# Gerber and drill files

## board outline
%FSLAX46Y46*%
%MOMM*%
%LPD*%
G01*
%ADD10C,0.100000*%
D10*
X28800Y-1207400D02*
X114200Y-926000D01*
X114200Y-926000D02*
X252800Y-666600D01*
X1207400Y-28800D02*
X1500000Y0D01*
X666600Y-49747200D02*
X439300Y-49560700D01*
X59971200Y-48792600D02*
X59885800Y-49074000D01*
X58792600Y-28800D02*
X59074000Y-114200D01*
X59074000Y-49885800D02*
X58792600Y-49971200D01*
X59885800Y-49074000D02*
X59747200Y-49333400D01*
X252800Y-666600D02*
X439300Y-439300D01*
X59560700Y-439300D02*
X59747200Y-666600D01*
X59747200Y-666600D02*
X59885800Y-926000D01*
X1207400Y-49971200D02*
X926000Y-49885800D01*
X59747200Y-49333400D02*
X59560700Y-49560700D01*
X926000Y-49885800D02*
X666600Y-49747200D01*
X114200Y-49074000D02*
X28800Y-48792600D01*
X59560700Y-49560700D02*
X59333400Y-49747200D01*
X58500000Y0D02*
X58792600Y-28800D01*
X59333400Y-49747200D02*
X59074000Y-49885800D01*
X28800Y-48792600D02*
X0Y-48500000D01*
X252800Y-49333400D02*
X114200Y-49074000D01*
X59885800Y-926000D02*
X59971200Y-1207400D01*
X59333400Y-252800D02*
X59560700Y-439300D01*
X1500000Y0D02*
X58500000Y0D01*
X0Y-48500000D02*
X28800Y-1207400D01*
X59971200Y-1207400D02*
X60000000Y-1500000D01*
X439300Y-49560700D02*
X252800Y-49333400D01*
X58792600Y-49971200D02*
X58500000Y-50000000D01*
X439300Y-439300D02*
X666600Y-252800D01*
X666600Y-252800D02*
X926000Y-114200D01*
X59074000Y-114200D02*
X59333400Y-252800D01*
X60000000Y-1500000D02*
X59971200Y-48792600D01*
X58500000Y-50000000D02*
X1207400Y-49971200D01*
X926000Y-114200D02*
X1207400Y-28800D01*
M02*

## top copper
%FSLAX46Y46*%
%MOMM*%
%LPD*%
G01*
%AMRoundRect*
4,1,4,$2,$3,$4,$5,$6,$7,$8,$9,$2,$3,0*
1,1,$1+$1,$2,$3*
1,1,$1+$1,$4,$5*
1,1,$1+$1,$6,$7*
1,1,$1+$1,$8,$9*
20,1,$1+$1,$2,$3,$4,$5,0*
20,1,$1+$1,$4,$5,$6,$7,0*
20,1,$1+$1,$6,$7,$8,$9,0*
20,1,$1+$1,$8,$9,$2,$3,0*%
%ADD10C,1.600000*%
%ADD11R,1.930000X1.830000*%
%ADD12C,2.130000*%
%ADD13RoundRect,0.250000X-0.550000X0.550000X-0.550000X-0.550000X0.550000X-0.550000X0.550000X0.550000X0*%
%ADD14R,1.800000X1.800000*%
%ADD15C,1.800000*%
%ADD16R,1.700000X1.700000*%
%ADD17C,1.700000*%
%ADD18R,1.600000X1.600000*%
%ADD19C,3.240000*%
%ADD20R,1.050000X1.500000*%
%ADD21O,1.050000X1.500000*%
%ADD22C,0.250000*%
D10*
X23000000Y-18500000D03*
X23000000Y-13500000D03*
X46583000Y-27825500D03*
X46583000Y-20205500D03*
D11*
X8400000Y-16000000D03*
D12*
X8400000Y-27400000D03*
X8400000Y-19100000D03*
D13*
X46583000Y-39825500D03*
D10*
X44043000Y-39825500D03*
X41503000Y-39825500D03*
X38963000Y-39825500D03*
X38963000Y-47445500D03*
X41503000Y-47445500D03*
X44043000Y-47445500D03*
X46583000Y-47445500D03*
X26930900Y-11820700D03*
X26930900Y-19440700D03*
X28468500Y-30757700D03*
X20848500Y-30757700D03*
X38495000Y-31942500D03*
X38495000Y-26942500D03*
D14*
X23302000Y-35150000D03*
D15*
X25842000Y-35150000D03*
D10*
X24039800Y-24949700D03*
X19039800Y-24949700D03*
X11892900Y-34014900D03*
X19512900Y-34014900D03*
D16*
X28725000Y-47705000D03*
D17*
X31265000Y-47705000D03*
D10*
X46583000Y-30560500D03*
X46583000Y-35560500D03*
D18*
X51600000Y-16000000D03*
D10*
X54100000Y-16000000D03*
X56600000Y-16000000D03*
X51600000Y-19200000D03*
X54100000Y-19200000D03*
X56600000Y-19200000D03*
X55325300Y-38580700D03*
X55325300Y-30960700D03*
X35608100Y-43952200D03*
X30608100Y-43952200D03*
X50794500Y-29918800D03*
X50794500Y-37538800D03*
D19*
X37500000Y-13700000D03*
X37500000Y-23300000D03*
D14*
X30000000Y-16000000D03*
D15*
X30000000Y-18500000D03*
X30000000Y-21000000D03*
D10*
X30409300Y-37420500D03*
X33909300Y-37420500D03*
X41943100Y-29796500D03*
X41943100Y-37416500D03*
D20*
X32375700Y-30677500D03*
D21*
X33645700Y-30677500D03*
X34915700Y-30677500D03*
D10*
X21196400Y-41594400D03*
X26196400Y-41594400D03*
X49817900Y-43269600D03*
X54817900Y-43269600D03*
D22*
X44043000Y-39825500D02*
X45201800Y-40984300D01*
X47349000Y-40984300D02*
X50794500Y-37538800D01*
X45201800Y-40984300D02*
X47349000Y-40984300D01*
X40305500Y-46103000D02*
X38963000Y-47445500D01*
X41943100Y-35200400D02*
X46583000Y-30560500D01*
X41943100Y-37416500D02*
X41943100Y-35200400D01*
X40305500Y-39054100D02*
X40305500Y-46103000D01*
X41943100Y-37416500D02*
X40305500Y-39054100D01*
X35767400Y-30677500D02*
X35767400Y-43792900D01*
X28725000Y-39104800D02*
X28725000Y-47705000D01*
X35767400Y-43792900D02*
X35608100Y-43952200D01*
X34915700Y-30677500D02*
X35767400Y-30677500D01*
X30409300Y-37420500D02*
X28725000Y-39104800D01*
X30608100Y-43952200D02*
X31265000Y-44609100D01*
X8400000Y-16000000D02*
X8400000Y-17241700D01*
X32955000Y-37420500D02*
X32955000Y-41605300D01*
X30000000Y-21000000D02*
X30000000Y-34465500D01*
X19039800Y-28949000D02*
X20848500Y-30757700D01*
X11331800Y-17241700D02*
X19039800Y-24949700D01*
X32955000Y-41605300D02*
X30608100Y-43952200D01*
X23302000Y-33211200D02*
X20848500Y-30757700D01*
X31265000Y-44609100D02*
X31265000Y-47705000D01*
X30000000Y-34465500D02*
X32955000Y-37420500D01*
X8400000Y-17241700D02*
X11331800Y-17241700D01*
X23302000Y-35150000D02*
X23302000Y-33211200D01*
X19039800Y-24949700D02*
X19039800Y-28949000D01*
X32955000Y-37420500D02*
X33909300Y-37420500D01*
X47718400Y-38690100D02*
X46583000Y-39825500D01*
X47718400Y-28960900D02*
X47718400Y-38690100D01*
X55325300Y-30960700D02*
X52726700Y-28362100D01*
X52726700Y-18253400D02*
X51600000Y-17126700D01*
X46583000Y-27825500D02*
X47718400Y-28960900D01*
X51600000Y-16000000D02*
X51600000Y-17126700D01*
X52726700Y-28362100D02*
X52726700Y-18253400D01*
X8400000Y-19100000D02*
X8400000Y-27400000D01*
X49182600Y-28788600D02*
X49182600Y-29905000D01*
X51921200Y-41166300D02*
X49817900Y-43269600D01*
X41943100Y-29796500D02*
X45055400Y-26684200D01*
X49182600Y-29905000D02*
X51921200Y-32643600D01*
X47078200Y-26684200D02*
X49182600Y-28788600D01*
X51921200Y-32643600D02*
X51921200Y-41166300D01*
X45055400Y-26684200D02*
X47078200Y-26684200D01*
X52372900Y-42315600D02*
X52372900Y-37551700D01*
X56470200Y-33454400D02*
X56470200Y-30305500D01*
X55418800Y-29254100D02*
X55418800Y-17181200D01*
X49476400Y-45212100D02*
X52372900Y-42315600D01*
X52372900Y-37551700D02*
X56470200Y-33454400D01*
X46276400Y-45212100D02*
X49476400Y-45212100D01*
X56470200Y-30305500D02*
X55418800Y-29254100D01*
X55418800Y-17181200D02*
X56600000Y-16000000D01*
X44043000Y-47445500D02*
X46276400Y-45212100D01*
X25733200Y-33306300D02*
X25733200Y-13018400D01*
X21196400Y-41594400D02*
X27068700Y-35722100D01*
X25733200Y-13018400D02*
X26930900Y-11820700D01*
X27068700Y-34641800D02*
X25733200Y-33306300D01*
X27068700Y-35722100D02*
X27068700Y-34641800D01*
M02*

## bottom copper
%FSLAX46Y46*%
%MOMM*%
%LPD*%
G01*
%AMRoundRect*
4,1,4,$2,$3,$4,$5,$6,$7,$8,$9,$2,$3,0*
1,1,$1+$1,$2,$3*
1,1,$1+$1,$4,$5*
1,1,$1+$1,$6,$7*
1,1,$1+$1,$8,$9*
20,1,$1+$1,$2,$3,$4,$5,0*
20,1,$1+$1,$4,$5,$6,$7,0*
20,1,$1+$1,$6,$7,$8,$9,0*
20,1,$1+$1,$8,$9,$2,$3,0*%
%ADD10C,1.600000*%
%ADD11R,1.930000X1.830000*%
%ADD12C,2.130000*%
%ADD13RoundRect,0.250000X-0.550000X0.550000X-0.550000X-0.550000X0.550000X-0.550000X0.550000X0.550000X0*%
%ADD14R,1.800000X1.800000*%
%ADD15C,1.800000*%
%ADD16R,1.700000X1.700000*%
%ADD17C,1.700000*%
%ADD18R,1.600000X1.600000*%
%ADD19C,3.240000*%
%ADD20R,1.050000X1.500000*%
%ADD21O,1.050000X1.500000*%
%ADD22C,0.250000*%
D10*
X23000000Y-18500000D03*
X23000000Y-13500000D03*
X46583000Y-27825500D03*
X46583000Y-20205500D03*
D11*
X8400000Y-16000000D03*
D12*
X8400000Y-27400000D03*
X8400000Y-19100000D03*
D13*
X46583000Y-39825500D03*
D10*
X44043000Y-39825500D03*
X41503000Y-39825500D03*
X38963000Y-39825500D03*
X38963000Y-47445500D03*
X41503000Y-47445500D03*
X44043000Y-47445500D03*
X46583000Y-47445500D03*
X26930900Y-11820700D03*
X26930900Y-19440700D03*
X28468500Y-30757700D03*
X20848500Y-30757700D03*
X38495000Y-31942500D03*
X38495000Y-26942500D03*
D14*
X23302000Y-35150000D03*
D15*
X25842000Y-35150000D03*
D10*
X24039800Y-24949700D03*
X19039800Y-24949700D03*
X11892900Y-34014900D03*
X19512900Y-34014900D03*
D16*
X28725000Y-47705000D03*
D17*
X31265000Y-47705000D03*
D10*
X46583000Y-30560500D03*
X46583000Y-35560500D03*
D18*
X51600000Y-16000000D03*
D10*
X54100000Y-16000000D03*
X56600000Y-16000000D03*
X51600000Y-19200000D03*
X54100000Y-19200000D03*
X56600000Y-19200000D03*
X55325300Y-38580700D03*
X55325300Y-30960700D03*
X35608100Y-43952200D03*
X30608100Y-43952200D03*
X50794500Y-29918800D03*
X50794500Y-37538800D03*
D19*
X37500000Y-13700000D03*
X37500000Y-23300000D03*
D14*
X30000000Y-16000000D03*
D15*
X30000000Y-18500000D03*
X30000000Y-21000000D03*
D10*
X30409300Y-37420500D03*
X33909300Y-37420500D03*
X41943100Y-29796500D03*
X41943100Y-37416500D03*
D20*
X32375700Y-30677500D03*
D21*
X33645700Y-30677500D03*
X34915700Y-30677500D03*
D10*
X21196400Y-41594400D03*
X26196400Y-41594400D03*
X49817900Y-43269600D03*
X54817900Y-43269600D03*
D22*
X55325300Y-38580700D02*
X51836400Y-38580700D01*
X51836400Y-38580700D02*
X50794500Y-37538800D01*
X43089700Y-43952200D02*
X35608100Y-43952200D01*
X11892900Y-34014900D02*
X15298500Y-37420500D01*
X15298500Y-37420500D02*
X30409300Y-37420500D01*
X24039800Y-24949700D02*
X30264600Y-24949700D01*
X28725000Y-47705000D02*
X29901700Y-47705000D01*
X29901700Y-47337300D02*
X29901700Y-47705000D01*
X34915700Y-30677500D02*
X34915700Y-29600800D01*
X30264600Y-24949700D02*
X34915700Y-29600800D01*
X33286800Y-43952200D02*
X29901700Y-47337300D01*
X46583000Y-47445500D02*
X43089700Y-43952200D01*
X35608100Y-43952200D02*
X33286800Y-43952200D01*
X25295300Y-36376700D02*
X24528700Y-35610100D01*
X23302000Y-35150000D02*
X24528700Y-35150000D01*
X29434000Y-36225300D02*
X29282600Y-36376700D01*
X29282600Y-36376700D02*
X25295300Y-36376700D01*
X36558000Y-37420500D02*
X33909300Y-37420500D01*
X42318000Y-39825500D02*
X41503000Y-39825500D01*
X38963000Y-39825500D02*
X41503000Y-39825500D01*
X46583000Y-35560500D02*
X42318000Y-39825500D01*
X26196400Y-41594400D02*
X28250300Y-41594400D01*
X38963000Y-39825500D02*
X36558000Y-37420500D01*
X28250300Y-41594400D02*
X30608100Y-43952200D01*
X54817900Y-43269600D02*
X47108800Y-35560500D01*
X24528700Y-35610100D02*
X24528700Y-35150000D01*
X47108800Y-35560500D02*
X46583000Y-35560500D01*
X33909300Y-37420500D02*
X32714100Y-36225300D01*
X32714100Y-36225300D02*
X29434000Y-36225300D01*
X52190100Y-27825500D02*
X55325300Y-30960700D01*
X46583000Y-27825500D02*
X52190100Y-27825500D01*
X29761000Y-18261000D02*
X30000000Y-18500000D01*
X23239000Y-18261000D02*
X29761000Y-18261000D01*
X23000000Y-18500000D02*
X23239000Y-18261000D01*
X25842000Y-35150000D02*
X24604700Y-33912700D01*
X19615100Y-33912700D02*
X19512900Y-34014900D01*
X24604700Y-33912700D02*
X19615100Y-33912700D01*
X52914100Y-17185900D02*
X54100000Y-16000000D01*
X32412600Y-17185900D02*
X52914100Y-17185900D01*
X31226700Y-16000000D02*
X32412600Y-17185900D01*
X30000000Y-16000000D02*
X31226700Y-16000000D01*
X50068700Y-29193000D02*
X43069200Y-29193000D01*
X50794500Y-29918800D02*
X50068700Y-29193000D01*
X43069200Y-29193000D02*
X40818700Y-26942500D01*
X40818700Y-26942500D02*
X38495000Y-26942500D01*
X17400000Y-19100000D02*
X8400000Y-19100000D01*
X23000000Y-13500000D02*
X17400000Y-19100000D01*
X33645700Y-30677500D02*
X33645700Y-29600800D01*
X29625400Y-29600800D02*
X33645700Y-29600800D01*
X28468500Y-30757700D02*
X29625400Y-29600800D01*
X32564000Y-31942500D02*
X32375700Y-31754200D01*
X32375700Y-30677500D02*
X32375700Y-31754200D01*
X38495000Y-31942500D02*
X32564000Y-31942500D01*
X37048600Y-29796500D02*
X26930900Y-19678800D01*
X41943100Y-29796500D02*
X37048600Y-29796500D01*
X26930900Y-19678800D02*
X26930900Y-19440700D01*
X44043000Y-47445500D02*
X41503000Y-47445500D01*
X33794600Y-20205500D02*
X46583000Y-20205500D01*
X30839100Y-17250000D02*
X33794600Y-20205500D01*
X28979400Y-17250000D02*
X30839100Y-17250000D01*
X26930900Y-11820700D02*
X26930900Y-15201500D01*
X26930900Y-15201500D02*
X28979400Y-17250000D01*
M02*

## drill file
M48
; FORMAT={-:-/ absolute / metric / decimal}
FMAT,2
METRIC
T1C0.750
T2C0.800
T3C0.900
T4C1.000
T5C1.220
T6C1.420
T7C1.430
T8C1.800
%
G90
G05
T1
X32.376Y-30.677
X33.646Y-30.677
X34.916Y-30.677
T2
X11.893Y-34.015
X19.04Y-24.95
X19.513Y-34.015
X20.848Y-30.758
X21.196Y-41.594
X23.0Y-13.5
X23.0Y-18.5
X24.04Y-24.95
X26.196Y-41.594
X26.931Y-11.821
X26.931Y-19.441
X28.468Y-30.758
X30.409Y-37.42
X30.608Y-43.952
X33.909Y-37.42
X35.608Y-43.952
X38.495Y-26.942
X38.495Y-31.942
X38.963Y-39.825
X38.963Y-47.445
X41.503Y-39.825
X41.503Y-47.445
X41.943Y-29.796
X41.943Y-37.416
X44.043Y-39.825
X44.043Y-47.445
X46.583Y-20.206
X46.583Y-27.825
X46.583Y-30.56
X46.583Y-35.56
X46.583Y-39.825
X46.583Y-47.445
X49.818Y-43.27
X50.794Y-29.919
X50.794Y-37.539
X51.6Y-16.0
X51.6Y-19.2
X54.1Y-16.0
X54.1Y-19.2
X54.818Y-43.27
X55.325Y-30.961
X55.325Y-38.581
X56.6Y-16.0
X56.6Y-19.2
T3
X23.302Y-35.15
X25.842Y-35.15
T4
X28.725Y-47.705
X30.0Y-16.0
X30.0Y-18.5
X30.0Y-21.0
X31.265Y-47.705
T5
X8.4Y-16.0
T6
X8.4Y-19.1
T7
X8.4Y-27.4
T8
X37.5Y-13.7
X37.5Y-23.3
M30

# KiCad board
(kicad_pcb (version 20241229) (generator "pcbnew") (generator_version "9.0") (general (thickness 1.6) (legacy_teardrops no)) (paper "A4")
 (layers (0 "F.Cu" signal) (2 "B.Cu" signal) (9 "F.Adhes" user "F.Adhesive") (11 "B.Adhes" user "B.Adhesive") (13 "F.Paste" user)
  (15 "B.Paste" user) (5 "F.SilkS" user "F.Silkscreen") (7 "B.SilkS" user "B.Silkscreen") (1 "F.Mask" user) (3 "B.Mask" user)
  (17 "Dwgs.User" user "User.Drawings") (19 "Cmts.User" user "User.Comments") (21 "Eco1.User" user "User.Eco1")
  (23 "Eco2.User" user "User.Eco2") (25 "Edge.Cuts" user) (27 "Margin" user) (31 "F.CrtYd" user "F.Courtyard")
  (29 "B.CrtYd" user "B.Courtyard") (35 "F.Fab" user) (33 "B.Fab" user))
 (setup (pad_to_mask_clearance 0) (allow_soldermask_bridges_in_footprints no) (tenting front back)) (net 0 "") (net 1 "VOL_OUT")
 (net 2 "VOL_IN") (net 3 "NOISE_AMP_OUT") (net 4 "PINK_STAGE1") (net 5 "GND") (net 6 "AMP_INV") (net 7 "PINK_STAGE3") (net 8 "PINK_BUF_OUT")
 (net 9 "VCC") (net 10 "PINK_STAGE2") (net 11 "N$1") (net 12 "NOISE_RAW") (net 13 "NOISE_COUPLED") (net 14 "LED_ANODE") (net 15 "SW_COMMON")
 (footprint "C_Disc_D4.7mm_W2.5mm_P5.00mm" (layer "F.Cu") (at 23 18.5 90)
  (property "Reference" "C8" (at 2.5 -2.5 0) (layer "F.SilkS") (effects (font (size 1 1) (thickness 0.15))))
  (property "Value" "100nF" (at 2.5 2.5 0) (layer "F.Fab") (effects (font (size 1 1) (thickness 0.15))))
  (pad "1" thru_hole circle (at 0 0 90) (size 1.6 1.6) (drill 0.8) (layers "*.Cu" "*.Mask") (remove_unused_layers no) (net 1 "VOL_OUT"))
  (pad "2" thru_hole circle (at 5 0 90) (size 1.6 1.6) (drill 0.8) (layers "*.Cu" "*.Mask") (remove_unused_layers no) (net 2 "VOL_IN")))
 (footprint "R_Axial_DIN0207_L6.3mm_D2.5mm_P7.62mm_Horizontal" (layer "F.Cu") (at 46.583 27.8255 90)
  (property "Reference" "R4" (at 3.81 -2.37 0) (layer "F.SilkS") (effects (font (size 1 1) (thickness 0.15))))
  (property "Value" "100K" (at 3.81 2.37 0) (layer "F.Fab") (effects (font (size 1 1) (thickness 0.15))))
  (pad "1" thru_hole circle (at 0 0 90) (size 1.6 1.6) (drill 0.8) (layers "*.Cu" "*.Mask") (remove_unused_layers no)
   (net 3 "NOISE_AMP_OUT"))
  (pad "2" thru_hole circle (at 7.62 0 90) (size 1.6 1.6) (drill 0.8) (layers "*.Cu" "*.Mask") (remove_unused_layers no)
   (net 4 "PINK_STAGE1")))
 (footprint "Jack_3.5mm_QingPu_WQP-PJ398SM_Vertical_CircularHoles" (layer "F.Cu") (at 8.4 16)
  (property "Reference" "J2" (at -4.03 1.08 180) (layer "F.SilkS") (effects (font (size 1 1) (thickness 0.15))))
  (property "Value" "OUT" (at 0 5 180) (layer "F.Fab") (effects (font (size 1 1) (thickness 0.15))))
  (pad "S" thru_hole rect (at 0 0 180) (size 1.93 1.83) (drill 1.22) (layers "*.Cu" "*.Mask") (remove_unused_layers no) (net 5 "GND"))
  (pad "T" thru_hole circle (at 0 11.4 180) (size 2.13 2.13) (drill 1.43) (layers "*.Cu" "*.Mask") (remove_unused_layers no)
   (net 2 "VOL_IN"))
  (pad "TN" thru_hole circle (at 0 3.1 180) (size 2.13 2.13) (drill 1.42) (layers "*.Cu" "*.Mask") (remove_unused_layers no)
   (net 2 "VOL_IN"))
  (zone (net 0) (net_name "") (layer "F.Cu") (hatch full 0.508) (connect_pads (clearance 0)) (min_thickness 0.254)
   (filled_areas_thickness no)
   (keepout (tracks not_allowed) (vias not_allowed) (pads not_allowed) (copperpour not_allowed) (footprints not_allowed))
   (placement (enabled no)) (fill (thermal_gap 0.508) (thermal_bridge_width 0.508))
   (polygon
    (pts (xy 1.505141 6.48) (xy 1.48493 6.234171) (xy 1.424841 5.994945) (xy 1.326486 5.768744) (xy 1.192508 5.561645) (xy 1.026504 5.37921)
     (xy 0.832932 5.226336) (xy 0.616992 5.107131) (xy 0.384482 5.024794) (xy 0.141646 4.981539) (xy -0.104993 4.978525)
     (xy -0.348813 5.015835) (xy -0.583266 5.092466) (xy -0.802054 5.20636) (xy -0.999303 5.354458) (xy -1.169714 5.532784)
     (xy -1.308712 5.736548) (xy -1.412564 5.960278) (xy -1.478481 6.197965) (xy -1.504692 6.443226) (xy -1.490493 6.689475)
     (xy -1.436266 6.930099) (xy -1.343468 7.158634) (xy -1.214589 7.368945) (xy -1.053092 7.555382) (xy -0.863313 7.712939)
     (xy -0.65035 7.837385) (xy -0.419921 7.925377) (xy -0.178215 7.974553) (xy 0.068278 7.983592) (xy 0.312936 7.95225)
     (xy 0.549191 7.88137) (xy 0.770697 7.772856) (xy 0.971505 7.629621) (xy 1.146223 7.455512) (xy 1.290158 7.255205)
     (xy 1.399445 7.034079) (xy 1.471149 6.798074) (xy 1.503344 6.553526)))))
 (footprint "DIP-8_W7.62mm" (layer "F.Cu") (at 46.583 39.8255 -90)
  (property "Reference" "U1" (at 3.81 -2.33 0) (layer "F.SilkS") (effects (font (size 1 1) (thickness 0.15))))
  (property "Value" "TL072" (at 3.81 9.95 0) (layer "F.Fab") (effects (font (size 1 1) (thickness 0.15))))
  (pad "1" thru_hole roundrect (at 0 0 270) (size 1.6 1.6) (drill 0.8) (layers "*.Cu" "*.Mask") (remove_unused_layers no)
   (roundrect_rratio 0.15625) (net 3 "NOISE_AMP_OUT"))
  (pad "2" thru_hole circle (at 0 2.54 270) (size 1.6 1.6) (drill 0.8) (layers "*.Cu" "*.Mask") (remove_unused_layers no) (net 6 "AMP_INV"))
  (pad "3" thru_hole circle (at 0 5.08 270) (size 1.6 1.6) (drill 0.8) (layers "*.Cu" "*.Mask") (remove_unused_layers no) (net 5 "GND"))
  (pad "4" thru_hole circle (at 0 7.62 270) (size 1.6 1.6) (drill 0.8) (layers "*.Cu" "*.Mask") (remove_unused_layers no) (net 5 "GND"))
  (pad "5" thru_hole circle (at 7.62 7.62 270) (size 1.6 1.6) (drill 0.8) (layers "*.Cu" "*.Mask") (remove_unused_layers no)
   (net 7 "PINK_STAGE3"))
  (pad "6" thru_hole circle (at 7.62 5.08 270) (size 1.6 1.6) (drill 0.8) (layers "*.Cu" "*.Mask") (remove_unused_layers no)
   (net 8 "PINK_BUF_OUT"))
  (pad "7" thru_hole circle (at 7.62 2.54 270) (size 1.6 1.6) (drill 0.8) (layers "*.Cu" "*.Mask") (remove_unused_layers no)
   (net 8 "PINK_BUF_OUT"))
  (pad "8" thru_hole circle (at 7.62 0 270) (size 1.6 1.6) (drill 0.8) (layers "*.Cu" "*.Mask") (remove_unused_layers no) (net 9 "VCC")))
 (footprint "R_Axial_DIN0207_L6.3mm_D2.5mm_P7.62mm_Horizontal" (layer "F.Cu") (at 26.9309 11.8207 -90)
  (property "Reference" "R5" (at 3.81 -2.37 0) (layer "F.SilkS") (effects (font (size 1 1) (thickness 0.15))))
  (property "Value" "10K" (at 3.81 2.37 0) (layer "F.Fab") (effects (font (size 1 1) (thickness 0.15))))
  (pad "1" thru_hole circle (at 0 0 270) (size 1.6 1.6) (drill 0.8) (layers "*.Cu" "*.Mask") (remove_unused_layers no) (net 4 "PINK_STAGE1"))
  (pad "2" thru_hole circle (at 7.62 0 270) (size 1.6 1.6) (drill 0.8) (layers "*.Cu" "*.Mask") (remove_unused_layers no)
   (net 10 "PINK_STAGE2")))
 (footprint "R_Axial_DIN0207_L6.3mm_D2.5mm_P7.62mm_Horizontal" (layer "F.Cu") (at 28.4685 30.7577 180)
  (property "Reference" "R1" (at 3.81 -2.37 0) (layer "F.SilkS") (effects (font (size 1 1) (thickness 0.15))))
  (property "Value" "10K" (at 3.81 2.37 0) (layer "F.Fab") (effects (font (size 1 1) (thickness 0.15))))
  (pad "1" thru_hole circle (at 0 0 180) (size 1.6 1.6) (drill 0.8) (layers "*.Cu" "*.Mask") (remove_unused_layers no) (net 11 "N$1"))
  (pad "2" thru_hole circle (at 7.62 0 180) (size 1.6 1.6) (drill 0.8) (layers "*.Cu" "*.Mask") (remove_unused_layers no) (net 5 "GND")))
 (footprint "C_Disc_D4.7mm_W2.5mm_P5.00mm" (layer "F.Cu") (at 38.495 31.9425 90)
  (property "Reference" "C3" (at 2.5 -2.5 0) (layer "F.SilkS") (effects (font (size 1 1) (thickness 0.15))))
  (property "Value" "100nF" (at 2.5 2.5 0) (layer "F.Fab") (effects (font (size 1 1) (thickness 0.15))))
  (pad "1" thru_hole circle (at 0 0 90) (size 1.6 1.6) (drill 0.8) (layers "*.Cu" "*.Mask") (remove_unused_layers no) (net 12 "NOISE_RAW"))
  (pad "2" thru_hole circle (at 5 0 90) (size 1.6 1.6) (drill 0.8) (layers "*.Cu" "*.Mask") (remove_unused_layers no)
   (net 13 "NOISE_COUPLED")))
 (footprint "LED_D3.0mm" (layer "F.Cu") (at 23.302 35.15)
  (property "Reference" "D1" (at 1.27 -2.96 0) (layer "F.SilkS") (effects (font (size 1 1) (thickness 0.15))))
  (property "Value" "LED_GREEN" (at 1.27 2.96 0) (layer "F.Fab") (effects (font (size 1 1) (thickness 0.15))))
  (pad "1" thru_hole rect (at 0 0) (size 1.8 1.8) (drill 0.9) (layers "*.Cu" "*.Mask") (remove_unused_layers no) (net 5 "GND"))
  (pad "2" thru_hole circle (at 2.54 0) (size 1.8 1.8) (drill 0.9) (layers "*.Cu" "*.Mask") (remove_unused_layers no) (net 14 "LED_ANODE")))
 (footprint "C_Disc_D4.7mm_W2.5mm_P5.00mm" (layer "F.Cu") (at 24.0398 24.9497 180)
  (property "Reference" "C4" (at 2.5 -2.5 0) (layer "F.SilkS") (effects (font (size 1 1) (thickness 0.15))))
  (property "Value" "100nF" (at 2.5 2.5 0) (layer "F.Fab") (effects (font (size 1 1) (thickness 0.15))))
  (pad "1" thru_hole circle (at 0 0 180) (size 1.6 1.6) (drill 0.8) (layers "*.Cu" "*.Mask") (remove_unused_layers no) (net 9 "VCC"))
  (pad "2" thru_hole circle (at 5 0 180) (size 1.6 1.6) (drill 0.8) (layers "*.Cu" "*.Mask") (remove_unused_layers no) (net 5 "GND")))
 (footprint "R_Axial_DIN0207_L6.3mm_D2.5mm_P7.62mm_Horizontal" (layer "F.Cu") (at 11.8929 34.0149)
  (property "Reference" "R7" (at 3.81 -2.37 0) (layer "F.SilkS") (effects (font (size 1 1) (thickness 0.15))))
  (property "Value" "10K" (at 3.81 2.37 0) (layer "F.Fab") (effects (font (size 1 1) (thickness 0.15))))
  (pad "1" thru_hole circle (at 0 0) (size 1.6 1.6) (drill 0.8) (layers "*.Cu" "*.Mask") (remove_unused_layers no) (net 9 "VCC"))
  (pad "2" thru_hole circle (at 7.62 0) (size 1.6 1.6) (drill 0.8) (layers "*.Cu" "*.Mask") (remove_unused_layers no) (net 14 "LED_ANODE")))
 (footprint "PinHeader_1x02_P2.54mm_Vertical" (layer "F.Cu") (at 28.725 47.705 90)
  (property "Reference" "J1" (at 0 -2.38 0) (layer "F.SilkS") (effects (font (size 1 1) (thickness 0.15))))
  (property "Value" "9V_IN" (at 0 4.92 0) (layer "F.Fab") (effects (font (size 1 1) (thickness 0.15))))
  (pad "1" thru_hole rect (at 0 0 90) (size 1.7 1.7) (drill 1) (layers "*.Cu" "*.Mask") (remove_unused_layers no) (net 9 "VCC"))
  (pad "2" thru_hole circle (at 0 2.54 90) (size 1.7 1.7) (drill 1) (layers "*.Cu" "*.Mask") (remove_unused_layers no) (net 5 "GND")))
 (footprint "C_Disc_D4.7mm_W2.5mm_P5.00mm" (layer "F.Cu") (at 46.583 30.5605 -90)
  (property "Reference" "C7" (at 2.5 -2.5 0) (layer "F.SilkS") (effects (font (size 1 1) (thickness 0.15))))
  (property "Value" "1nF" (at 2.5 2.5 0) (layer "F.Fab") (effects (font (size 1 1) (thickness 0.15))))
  (pad "1" thru_hole circle (at 0 0 270) (size 1.6 1.6) (drill 0.8) (layers "*.Cu" "*.Mask") (remove_unused_layers no) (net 7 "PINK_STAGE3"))
  (pad "2" thru_hole circle (at 5 0 270) (size 1.6 1.6) (drill 0.8) (layers "*.Cu" "*.Mask") (remove_unused_layers no) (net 5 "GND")))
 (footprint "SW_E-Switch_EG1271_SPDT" (layer "F.Cu") (at 51.6 16)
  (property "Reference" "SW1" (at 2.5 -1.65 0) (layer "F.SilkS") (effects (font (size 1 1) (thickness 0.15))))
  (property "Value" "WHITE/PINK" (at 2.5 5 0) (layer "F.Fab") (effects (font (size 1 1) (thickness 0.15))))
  (pad "1" thru_hole rect (at 0 0) (size 1.6 1.6) (drill 0.8) (layers "*.Cu" "*.Mask") (remove_unused_layers no) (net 3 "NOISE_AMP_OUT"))
  (pad "2" thru_hole circle (at 2.5 0) (size 1.6 1.6) (drill 0.8) (layers "*.Cu" "*.Mask") (remove_unused_layers no) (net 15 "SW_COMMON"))
  (pad "3" thru_hole circle (at 5 0) (size 1.6 1.6) (drill 0.8) (layers "*.Cu" "*.Mask") (remove_unused_layers no) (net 8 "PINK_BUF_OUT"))
  (pad "4" thru_hole circle (at 0 3.2) (size 1.6 1.6) (drill 0.8) (layers "*.Cu" "*.Mask") (remove_unused_layers no))
  (pad "5" thru_hole circle (at 2.5 3.2) (size 1.6 1.6) (drill 0.8) (layers "*.Cu" "*.Mask") (remove_unused_layers no))
  (pad "6" thru_hole circle (at 5 3.2) (size 1.6 1.6) (drill 0.8) (layers "*.Cu" "*.Mask") (remove_unused_layers no)))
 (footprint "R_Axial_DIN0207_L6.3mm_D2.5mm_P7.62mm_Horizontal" (layer "F.Cu") (at 55.3253 38.5807 90)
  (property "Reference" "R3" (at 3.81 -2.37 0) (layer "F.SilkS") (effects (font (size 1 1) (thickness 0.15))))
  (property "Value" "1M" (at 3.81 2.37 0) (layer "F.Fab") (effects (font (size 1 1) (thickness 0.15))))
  (pad "1" thru_hole circle (at 0 0 90) (size 1.6 1.6) (drill 0.8) (layers "*.Cu" "*.Mask") (remove_unused_layers no) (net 6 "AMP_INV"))
  (pad "2" thru_hole circle (at 7.62 0 90) (size 1.6 1.6) (drill 0.8) (layers "*.Cu" "*.Mask") (remove_unused_layers no)
   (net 3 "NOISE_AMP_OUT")))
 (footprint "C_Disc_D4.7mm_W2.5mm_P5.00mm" (layer "F.Cu") (at 35.6081 43.9522 180)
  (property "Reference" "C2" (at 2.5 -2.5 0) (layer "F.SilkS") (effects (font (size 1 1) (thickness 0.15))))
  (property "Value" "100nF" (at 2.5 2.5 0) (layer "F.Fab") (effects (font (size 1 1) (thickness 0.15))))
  (pad "1" thru_hole circle (at 0 0 180) (size 1.6 1.6) (drill 0.8) (layers "*.Cu" "*.Mask") (remove_unused_layers no) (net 9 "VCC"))
  (pad "2" thru_hole circle (at 5 0 180) (size 1.6 1.6) (drill 0.8) (layers "*.Cu" "*.Mask") (remove_unused_layers no) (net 5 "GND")))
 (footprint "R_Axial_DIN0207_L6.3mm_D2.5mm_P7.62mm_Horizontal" (layer "F.Cu") (at 50.7945 29.9188 -90)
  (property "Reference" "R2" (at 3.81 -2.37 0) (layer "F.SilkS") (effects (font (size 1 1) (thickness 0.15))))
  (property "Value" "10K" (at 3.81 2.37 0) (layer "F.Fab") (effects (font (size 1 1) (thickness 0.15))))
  (pad "1" thru_hole circle (at 0 0 270) (size 1.6 1.6) (drill 0.8) (layers "*.Cu" "*.Mask") (remove_unused_layers no)
   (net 13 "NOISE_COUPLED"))
  (pad "2" thru_hole circle (at 7.62 0 270) (size 1.6 1.6) (drill 0.8) (layers "*.Cu" "*.Mask") (remove_unused_layers no) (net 6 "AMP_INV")))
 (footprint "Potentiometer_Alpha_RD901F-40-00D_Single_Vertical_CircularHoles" (layer "F.Cu") (at 30 16)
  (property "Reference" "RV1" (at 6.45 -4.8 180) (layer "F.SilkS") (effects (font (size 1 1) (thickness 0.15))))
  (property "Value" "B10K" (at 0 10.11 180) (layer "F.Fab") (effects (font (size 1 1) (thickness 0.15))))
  (pad "" thru_hole circle (at 7.5 -2.3 90) (size 3.24 3.24) (drill 1.8) (layers "*.Cu" "*.Mask") (remove_unused_layers no))
  (pad "" thru_hole circle (at 7.5 7.3 90) (size 3.24 3.24) (drill 1.8) (layers "*.Cu" "*.Mask") (remove_unused_layers no))
  (pad "1" thru_hole rect (at 0 0 90) (size 1.8 1.8) (drill 1) (layers "*.Cu" "*.Mask") (remove_unused_layers no) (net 15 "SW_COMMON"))
  (pad "2" thru_hole circle (at 0 2.5 90) (size 1.8 1.8) (drill 1) (layers "*.Cu" "*.Mask") (remove_unused_layers no) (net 1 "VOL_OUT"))
  (pad "3" thru_hole circle (at 0 5 90) (size 1.8 1.8) (drill 1) (layers "*.Cu" "*.Mask") (remove_unused_layers no) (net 5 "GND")))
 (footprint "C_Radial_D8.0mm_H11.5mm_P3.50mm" (layer "F.Cu") (at 30.4093 37.4205)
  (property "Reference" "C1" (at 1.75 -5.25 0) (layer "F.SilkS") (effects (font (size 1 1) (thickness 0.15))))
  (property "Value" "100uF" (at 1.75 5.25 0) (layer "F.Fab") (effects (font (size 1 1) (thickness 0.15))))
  (pad "1" thru_hole circle (at 0 0) (size 1.6 1.6) (drill 0.8) (layers "*.Cu" "*.Mask") (remove_unused_layers no) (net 9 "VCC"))
  (pad "2" thru_hole circle (at 3.5 0) (size 1.6 1.6) (drill 0.8) (layers "*.Cu" "*.Mask") (remove_unused_layers no) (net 5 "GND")))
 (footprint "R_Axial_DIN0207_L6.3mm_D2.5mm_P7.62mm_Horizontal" (layer "F.Cu") (at 41.9431 29.7965 -90)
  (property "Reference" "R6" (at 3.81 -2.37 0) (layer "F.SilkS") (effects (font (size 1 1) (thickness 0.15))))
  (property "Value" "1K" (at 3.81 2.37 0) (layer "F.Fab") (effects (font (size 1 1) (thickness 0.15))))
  (pad "1" thru_hole circle (at 0 0 270) (size 1.6 1.6) (drill 0.8) (layers "*.Cu" "*.Mask") (remove_unused_layers no)
   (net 10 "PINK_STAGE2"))
  (pad "2" thru_hole circle (at 7.62 0 270) (size 1.6 1.6) (drill 0.8) (layers "*.Cu" "*.Mask") (remove_unused_layers no)
   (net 7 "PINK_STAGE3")))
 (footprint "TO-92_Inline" (layer "F.Cu") (at 32.3757 30.6775)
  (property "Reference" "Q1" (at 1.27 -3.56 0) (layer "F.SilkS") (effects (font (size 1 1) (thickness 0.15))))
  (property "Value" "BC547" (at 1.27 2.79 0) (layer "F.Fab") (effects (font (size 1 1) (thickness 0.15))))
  (pad "1" thru_hole rect (at 0 0) (size 1.05 1.5) (drill 0.75) (layers "*.Cu" "*.Mask") (remove_unused_layers no) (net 12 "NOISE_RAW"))
  (pad "2" thru_hole oval (at 1.27 0) (size 1.05 1.5) (drill 0.75) (layers "*.Cu" "*.Mask") (remove_unused_layers no) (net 11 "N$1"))
  (pad "3" thru_hole oval (at 2.54 0) (size 1.05 1.5) (drill 0.75) (layers "*.Cu" "*.Mask") (remove_unused_layers no) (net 9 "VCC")))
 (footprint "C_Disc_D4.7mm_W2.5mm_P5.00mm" (layer "F.Cu") (at 21.1964 41.5944)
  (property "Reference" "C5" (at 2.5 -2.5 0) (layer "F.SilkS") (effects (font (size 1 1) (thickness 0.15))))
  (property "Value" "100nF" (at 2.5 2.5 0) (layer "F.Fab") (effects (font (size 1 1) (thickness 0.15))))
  (pad "1" thru_hole circle (at 0 0) (size 1.6 1.6) (drill 0.8) (layers "*.Cu" "*.Mask") (remove_unused_layers no) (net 4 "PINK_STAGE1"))
  (pad "2" thru_hole circle (at 5 0) (size 1.6 1.6) (drill 0.8) (layers "*.Cu" "*.Mask") (remove_unused_layers no) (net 5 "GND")))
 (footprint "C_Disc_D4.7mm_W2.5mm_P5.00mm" (layer "F.Cu") (at 49.8179 43.2696)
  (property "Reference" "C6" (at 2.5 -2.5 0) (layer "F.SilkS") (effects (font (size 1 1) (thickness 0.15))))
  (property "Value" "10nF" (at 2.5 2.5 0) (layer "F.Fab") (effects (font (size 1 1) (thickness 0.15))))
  (pad "1" thru_hole circle (at 0 0) (size 1.6 1.6) (drill 0.8) (layers "*.Cu" "*.Mask") (remove_unused_layers no) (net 10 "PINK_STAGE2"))
  (pad "2" thru_hole circle (at 5 0) (size 1.6 1.6) (drill 0.8) (layers "*.Cu" "*.Mask") (remove_unused_layers no) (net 5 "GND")))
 (gr_line (start 0.0288 1.2074) (end 0.1142 0.926) (stroke (width 0.1) (type solid)) (layer "Edge.Cuts"))
 (gr_line (start 0.1142 0.926) (end 0.2528 0.6666) (stroke (width 0.1) (type solid)) (layer "Edge.Cuts"))
 (gr_line (start 1.2074 0.0288) (end 1.5 0) (stroke (width 0.1) (type solid)) (layer "Edge.Cuts"))
 (gr_line (start 0.6666 49.7472) (end 0.4393 49.5607) (stroke (width 0.1) (type solid)) (layer "Edge.Cuts"))
 (gr_line (start 59.9712 48.7926) (end 59.8858 49.074) (stroke (width 0.1) (type solid)) (layer "Edge.Cuts"))
 (gr_line (start 58.7926 0.0288) (end 59.074 0.1142) (stroke (width 0.1) (type solid)) (layer "Edge.Cuts"))
 (gr_line (start 59.074 49.8858) (end 58.7926 49.9712) (stroke (width 0.1) (type solid)) (layer "Edge.Cuts"))
 (gr_line (start 59.8858 49.074) (end 59.7472 49.3334) (stroke (width 0.1) (type solid)) (layer "Edge.Cuts"))
 (gr_line (start 0.2528 0.6666) (end 0.4393 0.4393) (stroke (width 0.1) (type solid)) (layer "Edge.Cuts"))
 (gr_line (start 59.5607 0.4393) (end 59.7472 0.6666) (stroke (width 0.1) (type solid)) (layer "Edge.Cuts"))
 (gr_line (start 59.7472 0.6666) (end 59.8858 0.926) (stroke (width 0.1) (type solid)) (layer "Edge.Cuts"))
 (gr_line (start 1.2074 49.9712) (end 0.926 49.8858) (stroke (width 0.1) (type solid)) (layer "Edge.Cuts"))
 (gr_line (start 59.7472 49.3334) (end 59.5607 49.5607) (stroke (width 0.1) (type solid)) (layer "Edge.Cuts"))
 (gr_line (start 0.926 49.8858) (end 0.6666 49.7472) (stroke (width 0.1) (type solid)) (layer "Edge.Cuts"))
 (gr_line (start 0.1142 49.074) (end 0.0288 48.7926) (stroke (width 0.1) (type solid)) (layer "Edge.Cuts"))
 (gr_line (start 59.5607 49.5607) (end 59.3334 49.7472) (stroke (width 0.1) (type solid)) (layer "Edge.Cuts"))
 (gr_line (start 58.5 0) (end 58.7926 0.0288) (stroke (width 0.1) (type solid)) (layer "Edge.Cuts"))
 (gr_line (start 59.3334 49.7472) (end 59.074 49.8858) (stroke (width 0.1) (type solid)) (layer "Edge.Cuts"))
 (gr_line (start 0.0288 48.7926) (end 0 48.5) (stroke (width 0.1) (type solid)) (layer "Edge.Cuts"))
 (gr_line (start 0.2528 49.3334) (end 0.1142 49.074) (stroke (width 0.1) (type solid)) (layer "Edge.Cuts"))
 (gr_line (start 59.8858 0.926) (end 59.9712 1.2074) (stroke (width 0.1) (type solid)) (layer "Edge.Cuts"))
 (gr_line (start 59.3334 0.2528) (end 59.5607 0.4393) (stroke (width 0.1) (type solid)) (layer "Edge.Cuts"))
 (gr_line (start 1.5 0) (end 58.5 0) (stroke (width 0.1) (type solid)) (layer "Edge.Cuts"))
 (gr_line (start 0 48.5) (end 0.0288 1.2074) (stroke (width 0.1) (type solid)) (layer "Edge.Cuts"))
 (gr_line (start 59.9712 1.2074) (end 60 1.5) (stroke (width 0.1) (type solid)) (layer "Edge.Cuts"))
 (gr_line (start 0.4393 49.5607) (end 0.2528 49.3334) (stroke (width 0.1) (type solid)) (layer "Edge.Cuts"))
 (gr_line (start 58.7926 49.9712) (end 58.5 50) (stroke (width 0.1) (type solid)) (layer "Edge.Cuts"))
 (gr_line (start 0.4393 0.4393) (end 0.6666 0.2528) (stroke (width 0.1) (type solid)) (layer "Edge.Cuts"))
 (gr_line (start 0.6666 0.2528) (end 0.926 0.1142) (stroke (width 0.1) (type solid)) (layer "Edge.Cuts"))
 (gr_line (start 59.074 0.1142) (end 59.3334 0.2528) (stroke (width 0.1) (type solid)) (layer "Edge.Cuts"))
 (gr_line (start 60 1.5) (end 59.9712 48.7926) (stroke (width 0.1) (type solid)) (layer "Edge.Cuts"))
 (gr_line (start 58.5 50) (end 1.2074 49.9712) (stroke (width 0.1) (type solid)) (layer "Edge.Cuts"))
 (gr_line (start 0.926 0.1142) (end 1.2074 0.0288) (stroke (width 0.1) (type solid)) (layer "Edge.Cuts"))
 (segment (start 44.043 39.8255) (end 45.2018 40.9843) (width 0.25) (layer "F.Cu") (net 6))
 (segment (start 47.349 40.9843) (end 50.7945 37.5388) (width 0.25) (layer "F.Cu") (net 6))
 (segment (start 45.2018 40.9843) (end 47.349 40.9843) (width 0.25) (layer "F.Cu") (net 6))
 (segment (start 55.3253 38.5807) (end 51.8364 38.5807) (width 0.25) (layer "B.Cu") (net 6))
 (segment (start 51.8364 38.5807) (end 50.7945 37.5388) (width 0.25) (layer "B.Cu") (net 6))
 (segment (start 40.3055 46.103) (end 38.963 47.4455) (width 0.25) (layer "F.Cu") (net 7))
 (segment (start 41.9431 35.2004) (end 46.583 30.5605) (width 0.25) (layer "F.Cu") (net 7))
 (segment (start 41.9431 37.4165) (end 41.9431 35.2004) (width 0.25) (layer "F.Cu") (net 7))
 (segment (start 40.3055 39.0541) (end 40.3055 46.103) (width 0.25) (layer "F.Cu") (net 7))
 (segment (start 41.9431 37.4165) (end 40.3055 39.0541) (width 0.25) (layer "F.Cu") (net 7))
 (segment (start 35.7674 30.6775) (end 35.7674 43.7929) (width 0.25) (layer "F.Cu") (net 9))
 (segment (start 28.725 39.1048) (end 28.725 47.705) (width 0.25) (layer "F.Cu") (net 9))
 (segment (start 35.7674 43.7929) (end 35.6081 43.9522) (width 0.25) (layer "F.Cu") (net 9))
 (segment (start 34.9157 30.6775) (end 35.7674 30.6775) (width 0.25) (layer "F.Cu") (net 9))
 (segment (start 30.4093 37.4205) (end 28.725 39.1048) (width 0.25) (layer "F.Cu") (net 9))
 (segment (start 43.0897 43.9522) (end 35.6081 43.9522) (width 0.25) (layer "B.Cu") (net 9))
 (segment (start 11.8929 34.0149) (end 15.2985 37.4205) (width 0.25) (layer "B.Cu") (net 9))
 (segment (start 15.2985 37.4205) (end 30.4093 37.4205) (width 0.25) (layer "B.Cu") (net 9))
 (segment (start 24.0398 24.9497) (end 30.2646 24.9497) (width 0.25) (layer "B.Cu") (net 9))
 (segment (start 28.725 47.705) (end 29.9017 47.705) (width 0.25) (layer "B.Cu") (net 9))
 (segment (start 29.9017 47.3373) (end 29.9017 47.705) (width 0.25) (layer "B.Cu") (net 9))
 (segment (start 34.9157 30.6775) (end 34.9157 29.6008) (width 0.25) (layer "B.Cu") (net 9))
 (segment (start 30.2646 24.9497) (end 34.9157 29.6008) (width 0.25) (layer "B.Cu") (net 9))
 (segment (start 33.2868 43.9522) (end 29.9017 47.3373) (width 0.25) (layer "B.Cu") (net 9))
 (segment (start 46.583 47.4455) (end 43.0897 43.9522) (width 0.25) (layer "B.Cu") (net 9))
 (segment (start 35.6081 43.9522) (end 33.2868 43.9522) (width 0.25) (layer "B.Cu") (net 9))
 (segment (start 30.6081 43.9522) (end 31.265 44.6091) (width 0.25) (layer "F.Cu") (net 5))
 (segment (start 8.4 16) (end 8.4 17.2417) (width 0.25) (layer "F.Cu") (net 5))
 (segment (start 32.955 37.4205) (end 32.955 41.6053) (width 0.25) (layer "F.Cu") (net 5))
 (segment (start 30 21) (end 30 34.4655) (width 0.25) (layer "F.Cu") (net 5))
 (segment (start 19.0398 28.949) (end 20.8485 30.7577) (width 0.25) (layer "F.Cu") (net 5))
 (segment (start 11.3318 17.2417) (end 19.0398 24.9497) (width 0.25) (layer "F.Cu") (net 5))
 (segment (start 32.955 41.6053) (end 30.6081 43.9522) (width 0.25) (layer "F.Cu") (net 5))
 (segment (start 23.302 33.2112) (end 20.8485 30.7577) (width 0.25) (layer "F.Cu") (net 5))
 (segment (start 31.265 44.6091) (end 31.265 47.705) (width 0.25) (layer "F.Cu") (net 5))
 (segment (start 30 34.4655) (end 32.955 37.4205) (width 0.25) (layer "F.Cu") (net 5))
 (segment (start 8.4 17.2417) (end 11.3318 17.2417) (width 0.25) (layer "F.Cu") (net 5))
 (segment (start 23.302 35.15) (end 23.302 33.2112) (width 0.25) (layer "F.Cu") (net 5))
 (segment (start 19.0398 24.9497) (end 19.0398 28.949) (width 0.25) (layer "F.Cu") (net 5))
 (segment (start 32.955 37.4205) (end 33.9093 37.4205) (width 0.25) (layer "F.Cu") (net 5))
 (segment (start 25.2953 36.3767) (end 24.5287 35.6101) (width 0.25) (layer "B.Cu") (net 5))
 (segment (start 23.302 35.15) (end 24.5287 35.15) (width 0.25) (layer "B.Cu") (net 5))
 (segment (start 29.434 36.2253) (end 29.2826 36.3767) (width 0.25) (layer "B.Cu") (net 5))
 (segment (start 29.2826 36.3767) (end 25.2953 36.3767) (width 0.25) (layer "B.Cu") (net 5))
 (segment (start 36.558 37.4205) (end 33.9093 37.4205) (width 0.25) (layer "B.Cu") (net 5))
 (segment (start 42.318 39.8255) (end 41.503 39.8255) (width 0.25) (layer "B.Cu") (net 5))
 (segment (start 38.963 39.8255) (end 41.503 39.8255) (width 0.25) (layer "B.Cu") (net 5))
 (segment (start 46.583 35.5605) (end 42.318 39.8255) (width 0.25) (layer "B.Cu") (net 5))
 (segment (start 26.1964 41.5944) (end 28.2503 41.5944) (width 0.25) (layer "B.Cu") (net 5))
 (segment (start 38.963 39.8255) (end 36.558 37.4205) (width 0.25) (layer "B.Cu") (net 5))
 (segment (start 28.2503 41.5944) (end 30.6081 43.9522) (width 0.25) (layer "B.Cu") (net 5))
 (segment (start 54.8179 43.2696) (end 47.1088 35.5605) (width 0.25) (layer "B.Cu") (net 5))
 (segment (start 24.5287 35.6101) (end 24.5287 35.15) (width 0.25) (layer "B.Cu") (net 5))
 (segment (start 47.1088 35.5605) (end 46.583 35.5605) (width 0.25) (layer "B.Cu") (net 5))
 (segment (start 33.9093 37.4205) (end 32.7141 36.2253) (width 0.25) (layer "B.Cu") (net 5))
 (segment (start 32.7141 36.2253) (end 29.434 36.2253) (width 0.25) (layer "B.Cu") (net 5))
 (segment (start 47.7184 38.6901) (end 46.583 39.8255) (width 0.25) (layer "F.Cu") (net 3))
 (segment (start 47.7184 28.9609) (end 47.7184 38.6901) (width 0.25) (layer "F.Cu") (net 3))
 (segment (start 55.3253 30.9607) (end 52.7267 28.3621) (width 0.25) (layer "F.Cu") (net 3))
 (segment (start 52.7267 18.2534) (end 51.6 17.1267) (width 0.25) (layer "F.Cu") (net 3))
 (segment (start 46.583 27.8255) (end 47.7184 28.9609) (width 0.25) (layer "F.Cu") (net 3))
 (segment (start 51.6 16) (end 51.6 17.1267) (width 0.25) (layer "F.Cu") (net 3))
 (segment (start 52.7267 28.3621) (end 52.7267 18.2534) (width 0.25) (layer "F.Cu") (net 3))
 (segment (start 52.1901 27.8255) (end 55.3253 30.9607) (width 0.25) (layer "B.Cu") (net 3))
 (segment (start 46.583 27.8255) (end 52.1901 27.8255) (width 0.25) (layer "B.Cu") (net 3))
 (segment (start 29.761 18.261) (end 30 18.5) (width 0.25) (layer "B.Cu") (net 1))
 (segment (start 23.239 18.261) (end 29.761 18.261) (width 0.25) (layer "B.Cu") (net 1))
 (segment (start 23 18.5) (end 23.239 18.261) (width 0.25) (layer "B.Cu") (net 1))
 (segment (start 25.842 35.15) (end 24.6047 33.9127) (width 0.25) (layer "B.Cu") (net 14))
 (segment (start 19.6151 33.9127) (end 19.5129 34.0149) (width 0.25) (layer "B.Cu") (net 14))
 (segment (start 24.6047 33.9127) (end 19.6151 33.9127) (width 0.25) (layer "B.Cu") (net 14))
 (segment (start 52.9141 17.1859) (end 54.1 16) (width 0.25) (layer "B.Cu") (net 15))
 (segment (start 32.4126 17.1859) (end 52.9141 17.1859) (width 0.25) (layer "B.Cu") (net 15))
 (segment (start 31.2267 16) (end 32.4126 17.1859) (width 0.25) (layer "B.Cu") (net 15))
 (segment (start 30 16) (end 31.2267 16) (width 0.25) (layer "B.Cu") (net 15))
 (segment (start 50.0687 29.193) (end 43.0692 29.193) (width 0.25) (layer "B.Cu") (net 13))
 (segment (start 50.7945 29.9188) (end 50.0687 29.193) (width 0.25) (layer "B.Cu") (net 13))
 (segment (start 43.0692 29.193) (end 40.8187 26.9425) (width 0.25) (layer "B.Cu") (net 13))
 (segment (start 40.8187 26.9425) (end 38.495 26.9425) (width 0.25) (layer "B.Cu") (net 13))
 (segment (start 8.4 19.1) (end 8.4 27.4) (width 0.25) (layer "F.Cu") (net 2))
 (segment (start 17.4 19.1) (end 8.4 19.1) (width 0.25) (layer "B.Cu") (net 2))
 (segment (start 23 13.5) (end 17.4 19.1) (width 0.25) (layer "B.Cu") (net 2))
 (segment (start 33.6457 30.6775) (end 33.6457 29.6008) (width 0.25) (layer "B.Cu") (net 11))
 (segment (start 29.6254 29.6008) (end 33.6457 29.6008) (width 0.25) (layer "B.Cu") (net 11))
 (segment (start 28.4685 30.7577) (end 29.6254 29.6008) (width 0.25) (layer "B.Cu") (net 11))
 (segment (start 32.564 31.9425) (end 32.3757 31.7542) (width 0.25) (layer "B.Cu") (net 12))
 (segment (start 32.3757 30.6775) (end 32.3757 31.7542) (width 0.25) (layer "B.Cu") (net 12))
 (segment (start 38.495 31.9425) (end 32.564 31.9425) (width 0.25) (layer "B.Cu") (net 12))
 (segment (start 49.1826 28.7886) (end 49.1826 29.905) (width 0.25) (layer "F.Cu") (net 10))
 (segment (start 51.9212 41.1663) (end 49.8179 43.2696) (width 0.25) (layer "F.Cu") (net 10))
 (segment (start 41.9431 29.7965) (end 45.0554 26.6842) (width 0.25) (layer "F.Cu") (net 10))
 (segment (start 49.1826 29.905) (end 51.9212 32.6436) (width 0.25) (layer "F.Cu") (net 10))
 (segment (start 47.0782 26.6842) (end 49.1826 28.7886) (width 0.25) (layer "F.Cu") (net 10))
 (segment (start 51.9212 32.6436) (end 51.9212 41.1663) (width 0.25) (layer "F.Cu") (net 10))
 (segment (start 45.0554 26.6842) (end 47.0782 26.6842) (width 0.25) (layer "F.Cu") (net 10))
 (segment (start 37.0486 29.7965) (end 26.9309 19.6788) (width 0.25) (layer "B.Cu") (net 10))
 (segment (start 41.9431 29.7965) (end 37.0486 29.7965) (width 0.25) (layer "B.Cu") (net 10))
 (segment (start 26.9309 19.6788) (end 26.9309 19.4407) (width 0.25) (layer "B.Cu") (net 10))
 (segment (start 52.3729 42.3156) (end 52.3729 37.5517) (width 0.25) (layer "F.Cu") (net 8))
 (segment (start 56.4702 33.4544) (end 56.4702 30.3055) (width 0.25) (layer "F.Cu") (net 8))
 (segment (start 55.4188 29.2541) (end 55.4188 17.1812) (width 0.25) (layer "F.Cu") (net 8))
 (segment (start 49.4764 45.2121) (end 52.3729 42.3156) (width 0.25) (layer "F.Cu") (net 8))
 (segment (start 52.3729 37.5517) (end 56.4702 33.4544) (width 0.25) (layer "F.Cu") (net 8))
 (segment (start 46.2764 45.2121) (end 49.4764 45.2121) (width 0.25) (layer "F.Cu") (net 8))
 (segment (start 56.4702 30.3055) (end 55.4188 29.2541) (width 0.25) (layer "F.Cu") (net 8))
 (segment (start 55.4188 17.1812) (end 56.6 16) (width 0.25) (layer "F.Cu") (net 8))
 (segment (start 44.043 47.4455) (end 46.2764 45.2121) (width 0.25) (layer "F.Cu") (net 8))
 (segment (start 44.043 47.4455) (end 41.503 47.4455) (width 0.25) (layer "B.Cu") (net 8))
 (segment (start 25.7332 33.3063) (end 25.7332 13.0184) (width 0.25) (layer "F.Cu") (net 4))
 (segment (start 21.1964 41.5944) (end 27.0687 35.7221) (width 0.25) (layer "F.Cu") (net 4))
 (segment (start 25.7332 13.0184) (end 26.9309 11.8207) (width 0.25) (layer "F.Cu") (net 4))
 (segment (start 27.0687 34.6418) (end 25.7332 33.3063) (width 0.25) (layer "F.Cu") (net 4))
 (segment (start 27.0687 35.7221) (end 27.0687 34.6418) (width 0.25) (layer "F.Cu") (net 4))
 (segment (start 33.7946 20.2055) (end 46.583 20.2055) (width 0.25) (layer "B.Cu") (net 4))
 (segment (start 30.8391 17.25) (end 33.7946 20.2055) (width 0.25) (layer "B.Cu") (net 4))
 (segment (start 28.9794 17.25) (end 30.8391 17.25) (width 0.25) (layer "B.Cu") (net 4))
 (segment (start 26.9309 11.8207) (end 26.9309 15.2015) (width 0.25) (layer "B.Cu") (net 4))
 (segment (start 26.9309 15.2015) (end 28.9794 17.25) (width 0.25) (layer "B.Cu") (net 4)))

